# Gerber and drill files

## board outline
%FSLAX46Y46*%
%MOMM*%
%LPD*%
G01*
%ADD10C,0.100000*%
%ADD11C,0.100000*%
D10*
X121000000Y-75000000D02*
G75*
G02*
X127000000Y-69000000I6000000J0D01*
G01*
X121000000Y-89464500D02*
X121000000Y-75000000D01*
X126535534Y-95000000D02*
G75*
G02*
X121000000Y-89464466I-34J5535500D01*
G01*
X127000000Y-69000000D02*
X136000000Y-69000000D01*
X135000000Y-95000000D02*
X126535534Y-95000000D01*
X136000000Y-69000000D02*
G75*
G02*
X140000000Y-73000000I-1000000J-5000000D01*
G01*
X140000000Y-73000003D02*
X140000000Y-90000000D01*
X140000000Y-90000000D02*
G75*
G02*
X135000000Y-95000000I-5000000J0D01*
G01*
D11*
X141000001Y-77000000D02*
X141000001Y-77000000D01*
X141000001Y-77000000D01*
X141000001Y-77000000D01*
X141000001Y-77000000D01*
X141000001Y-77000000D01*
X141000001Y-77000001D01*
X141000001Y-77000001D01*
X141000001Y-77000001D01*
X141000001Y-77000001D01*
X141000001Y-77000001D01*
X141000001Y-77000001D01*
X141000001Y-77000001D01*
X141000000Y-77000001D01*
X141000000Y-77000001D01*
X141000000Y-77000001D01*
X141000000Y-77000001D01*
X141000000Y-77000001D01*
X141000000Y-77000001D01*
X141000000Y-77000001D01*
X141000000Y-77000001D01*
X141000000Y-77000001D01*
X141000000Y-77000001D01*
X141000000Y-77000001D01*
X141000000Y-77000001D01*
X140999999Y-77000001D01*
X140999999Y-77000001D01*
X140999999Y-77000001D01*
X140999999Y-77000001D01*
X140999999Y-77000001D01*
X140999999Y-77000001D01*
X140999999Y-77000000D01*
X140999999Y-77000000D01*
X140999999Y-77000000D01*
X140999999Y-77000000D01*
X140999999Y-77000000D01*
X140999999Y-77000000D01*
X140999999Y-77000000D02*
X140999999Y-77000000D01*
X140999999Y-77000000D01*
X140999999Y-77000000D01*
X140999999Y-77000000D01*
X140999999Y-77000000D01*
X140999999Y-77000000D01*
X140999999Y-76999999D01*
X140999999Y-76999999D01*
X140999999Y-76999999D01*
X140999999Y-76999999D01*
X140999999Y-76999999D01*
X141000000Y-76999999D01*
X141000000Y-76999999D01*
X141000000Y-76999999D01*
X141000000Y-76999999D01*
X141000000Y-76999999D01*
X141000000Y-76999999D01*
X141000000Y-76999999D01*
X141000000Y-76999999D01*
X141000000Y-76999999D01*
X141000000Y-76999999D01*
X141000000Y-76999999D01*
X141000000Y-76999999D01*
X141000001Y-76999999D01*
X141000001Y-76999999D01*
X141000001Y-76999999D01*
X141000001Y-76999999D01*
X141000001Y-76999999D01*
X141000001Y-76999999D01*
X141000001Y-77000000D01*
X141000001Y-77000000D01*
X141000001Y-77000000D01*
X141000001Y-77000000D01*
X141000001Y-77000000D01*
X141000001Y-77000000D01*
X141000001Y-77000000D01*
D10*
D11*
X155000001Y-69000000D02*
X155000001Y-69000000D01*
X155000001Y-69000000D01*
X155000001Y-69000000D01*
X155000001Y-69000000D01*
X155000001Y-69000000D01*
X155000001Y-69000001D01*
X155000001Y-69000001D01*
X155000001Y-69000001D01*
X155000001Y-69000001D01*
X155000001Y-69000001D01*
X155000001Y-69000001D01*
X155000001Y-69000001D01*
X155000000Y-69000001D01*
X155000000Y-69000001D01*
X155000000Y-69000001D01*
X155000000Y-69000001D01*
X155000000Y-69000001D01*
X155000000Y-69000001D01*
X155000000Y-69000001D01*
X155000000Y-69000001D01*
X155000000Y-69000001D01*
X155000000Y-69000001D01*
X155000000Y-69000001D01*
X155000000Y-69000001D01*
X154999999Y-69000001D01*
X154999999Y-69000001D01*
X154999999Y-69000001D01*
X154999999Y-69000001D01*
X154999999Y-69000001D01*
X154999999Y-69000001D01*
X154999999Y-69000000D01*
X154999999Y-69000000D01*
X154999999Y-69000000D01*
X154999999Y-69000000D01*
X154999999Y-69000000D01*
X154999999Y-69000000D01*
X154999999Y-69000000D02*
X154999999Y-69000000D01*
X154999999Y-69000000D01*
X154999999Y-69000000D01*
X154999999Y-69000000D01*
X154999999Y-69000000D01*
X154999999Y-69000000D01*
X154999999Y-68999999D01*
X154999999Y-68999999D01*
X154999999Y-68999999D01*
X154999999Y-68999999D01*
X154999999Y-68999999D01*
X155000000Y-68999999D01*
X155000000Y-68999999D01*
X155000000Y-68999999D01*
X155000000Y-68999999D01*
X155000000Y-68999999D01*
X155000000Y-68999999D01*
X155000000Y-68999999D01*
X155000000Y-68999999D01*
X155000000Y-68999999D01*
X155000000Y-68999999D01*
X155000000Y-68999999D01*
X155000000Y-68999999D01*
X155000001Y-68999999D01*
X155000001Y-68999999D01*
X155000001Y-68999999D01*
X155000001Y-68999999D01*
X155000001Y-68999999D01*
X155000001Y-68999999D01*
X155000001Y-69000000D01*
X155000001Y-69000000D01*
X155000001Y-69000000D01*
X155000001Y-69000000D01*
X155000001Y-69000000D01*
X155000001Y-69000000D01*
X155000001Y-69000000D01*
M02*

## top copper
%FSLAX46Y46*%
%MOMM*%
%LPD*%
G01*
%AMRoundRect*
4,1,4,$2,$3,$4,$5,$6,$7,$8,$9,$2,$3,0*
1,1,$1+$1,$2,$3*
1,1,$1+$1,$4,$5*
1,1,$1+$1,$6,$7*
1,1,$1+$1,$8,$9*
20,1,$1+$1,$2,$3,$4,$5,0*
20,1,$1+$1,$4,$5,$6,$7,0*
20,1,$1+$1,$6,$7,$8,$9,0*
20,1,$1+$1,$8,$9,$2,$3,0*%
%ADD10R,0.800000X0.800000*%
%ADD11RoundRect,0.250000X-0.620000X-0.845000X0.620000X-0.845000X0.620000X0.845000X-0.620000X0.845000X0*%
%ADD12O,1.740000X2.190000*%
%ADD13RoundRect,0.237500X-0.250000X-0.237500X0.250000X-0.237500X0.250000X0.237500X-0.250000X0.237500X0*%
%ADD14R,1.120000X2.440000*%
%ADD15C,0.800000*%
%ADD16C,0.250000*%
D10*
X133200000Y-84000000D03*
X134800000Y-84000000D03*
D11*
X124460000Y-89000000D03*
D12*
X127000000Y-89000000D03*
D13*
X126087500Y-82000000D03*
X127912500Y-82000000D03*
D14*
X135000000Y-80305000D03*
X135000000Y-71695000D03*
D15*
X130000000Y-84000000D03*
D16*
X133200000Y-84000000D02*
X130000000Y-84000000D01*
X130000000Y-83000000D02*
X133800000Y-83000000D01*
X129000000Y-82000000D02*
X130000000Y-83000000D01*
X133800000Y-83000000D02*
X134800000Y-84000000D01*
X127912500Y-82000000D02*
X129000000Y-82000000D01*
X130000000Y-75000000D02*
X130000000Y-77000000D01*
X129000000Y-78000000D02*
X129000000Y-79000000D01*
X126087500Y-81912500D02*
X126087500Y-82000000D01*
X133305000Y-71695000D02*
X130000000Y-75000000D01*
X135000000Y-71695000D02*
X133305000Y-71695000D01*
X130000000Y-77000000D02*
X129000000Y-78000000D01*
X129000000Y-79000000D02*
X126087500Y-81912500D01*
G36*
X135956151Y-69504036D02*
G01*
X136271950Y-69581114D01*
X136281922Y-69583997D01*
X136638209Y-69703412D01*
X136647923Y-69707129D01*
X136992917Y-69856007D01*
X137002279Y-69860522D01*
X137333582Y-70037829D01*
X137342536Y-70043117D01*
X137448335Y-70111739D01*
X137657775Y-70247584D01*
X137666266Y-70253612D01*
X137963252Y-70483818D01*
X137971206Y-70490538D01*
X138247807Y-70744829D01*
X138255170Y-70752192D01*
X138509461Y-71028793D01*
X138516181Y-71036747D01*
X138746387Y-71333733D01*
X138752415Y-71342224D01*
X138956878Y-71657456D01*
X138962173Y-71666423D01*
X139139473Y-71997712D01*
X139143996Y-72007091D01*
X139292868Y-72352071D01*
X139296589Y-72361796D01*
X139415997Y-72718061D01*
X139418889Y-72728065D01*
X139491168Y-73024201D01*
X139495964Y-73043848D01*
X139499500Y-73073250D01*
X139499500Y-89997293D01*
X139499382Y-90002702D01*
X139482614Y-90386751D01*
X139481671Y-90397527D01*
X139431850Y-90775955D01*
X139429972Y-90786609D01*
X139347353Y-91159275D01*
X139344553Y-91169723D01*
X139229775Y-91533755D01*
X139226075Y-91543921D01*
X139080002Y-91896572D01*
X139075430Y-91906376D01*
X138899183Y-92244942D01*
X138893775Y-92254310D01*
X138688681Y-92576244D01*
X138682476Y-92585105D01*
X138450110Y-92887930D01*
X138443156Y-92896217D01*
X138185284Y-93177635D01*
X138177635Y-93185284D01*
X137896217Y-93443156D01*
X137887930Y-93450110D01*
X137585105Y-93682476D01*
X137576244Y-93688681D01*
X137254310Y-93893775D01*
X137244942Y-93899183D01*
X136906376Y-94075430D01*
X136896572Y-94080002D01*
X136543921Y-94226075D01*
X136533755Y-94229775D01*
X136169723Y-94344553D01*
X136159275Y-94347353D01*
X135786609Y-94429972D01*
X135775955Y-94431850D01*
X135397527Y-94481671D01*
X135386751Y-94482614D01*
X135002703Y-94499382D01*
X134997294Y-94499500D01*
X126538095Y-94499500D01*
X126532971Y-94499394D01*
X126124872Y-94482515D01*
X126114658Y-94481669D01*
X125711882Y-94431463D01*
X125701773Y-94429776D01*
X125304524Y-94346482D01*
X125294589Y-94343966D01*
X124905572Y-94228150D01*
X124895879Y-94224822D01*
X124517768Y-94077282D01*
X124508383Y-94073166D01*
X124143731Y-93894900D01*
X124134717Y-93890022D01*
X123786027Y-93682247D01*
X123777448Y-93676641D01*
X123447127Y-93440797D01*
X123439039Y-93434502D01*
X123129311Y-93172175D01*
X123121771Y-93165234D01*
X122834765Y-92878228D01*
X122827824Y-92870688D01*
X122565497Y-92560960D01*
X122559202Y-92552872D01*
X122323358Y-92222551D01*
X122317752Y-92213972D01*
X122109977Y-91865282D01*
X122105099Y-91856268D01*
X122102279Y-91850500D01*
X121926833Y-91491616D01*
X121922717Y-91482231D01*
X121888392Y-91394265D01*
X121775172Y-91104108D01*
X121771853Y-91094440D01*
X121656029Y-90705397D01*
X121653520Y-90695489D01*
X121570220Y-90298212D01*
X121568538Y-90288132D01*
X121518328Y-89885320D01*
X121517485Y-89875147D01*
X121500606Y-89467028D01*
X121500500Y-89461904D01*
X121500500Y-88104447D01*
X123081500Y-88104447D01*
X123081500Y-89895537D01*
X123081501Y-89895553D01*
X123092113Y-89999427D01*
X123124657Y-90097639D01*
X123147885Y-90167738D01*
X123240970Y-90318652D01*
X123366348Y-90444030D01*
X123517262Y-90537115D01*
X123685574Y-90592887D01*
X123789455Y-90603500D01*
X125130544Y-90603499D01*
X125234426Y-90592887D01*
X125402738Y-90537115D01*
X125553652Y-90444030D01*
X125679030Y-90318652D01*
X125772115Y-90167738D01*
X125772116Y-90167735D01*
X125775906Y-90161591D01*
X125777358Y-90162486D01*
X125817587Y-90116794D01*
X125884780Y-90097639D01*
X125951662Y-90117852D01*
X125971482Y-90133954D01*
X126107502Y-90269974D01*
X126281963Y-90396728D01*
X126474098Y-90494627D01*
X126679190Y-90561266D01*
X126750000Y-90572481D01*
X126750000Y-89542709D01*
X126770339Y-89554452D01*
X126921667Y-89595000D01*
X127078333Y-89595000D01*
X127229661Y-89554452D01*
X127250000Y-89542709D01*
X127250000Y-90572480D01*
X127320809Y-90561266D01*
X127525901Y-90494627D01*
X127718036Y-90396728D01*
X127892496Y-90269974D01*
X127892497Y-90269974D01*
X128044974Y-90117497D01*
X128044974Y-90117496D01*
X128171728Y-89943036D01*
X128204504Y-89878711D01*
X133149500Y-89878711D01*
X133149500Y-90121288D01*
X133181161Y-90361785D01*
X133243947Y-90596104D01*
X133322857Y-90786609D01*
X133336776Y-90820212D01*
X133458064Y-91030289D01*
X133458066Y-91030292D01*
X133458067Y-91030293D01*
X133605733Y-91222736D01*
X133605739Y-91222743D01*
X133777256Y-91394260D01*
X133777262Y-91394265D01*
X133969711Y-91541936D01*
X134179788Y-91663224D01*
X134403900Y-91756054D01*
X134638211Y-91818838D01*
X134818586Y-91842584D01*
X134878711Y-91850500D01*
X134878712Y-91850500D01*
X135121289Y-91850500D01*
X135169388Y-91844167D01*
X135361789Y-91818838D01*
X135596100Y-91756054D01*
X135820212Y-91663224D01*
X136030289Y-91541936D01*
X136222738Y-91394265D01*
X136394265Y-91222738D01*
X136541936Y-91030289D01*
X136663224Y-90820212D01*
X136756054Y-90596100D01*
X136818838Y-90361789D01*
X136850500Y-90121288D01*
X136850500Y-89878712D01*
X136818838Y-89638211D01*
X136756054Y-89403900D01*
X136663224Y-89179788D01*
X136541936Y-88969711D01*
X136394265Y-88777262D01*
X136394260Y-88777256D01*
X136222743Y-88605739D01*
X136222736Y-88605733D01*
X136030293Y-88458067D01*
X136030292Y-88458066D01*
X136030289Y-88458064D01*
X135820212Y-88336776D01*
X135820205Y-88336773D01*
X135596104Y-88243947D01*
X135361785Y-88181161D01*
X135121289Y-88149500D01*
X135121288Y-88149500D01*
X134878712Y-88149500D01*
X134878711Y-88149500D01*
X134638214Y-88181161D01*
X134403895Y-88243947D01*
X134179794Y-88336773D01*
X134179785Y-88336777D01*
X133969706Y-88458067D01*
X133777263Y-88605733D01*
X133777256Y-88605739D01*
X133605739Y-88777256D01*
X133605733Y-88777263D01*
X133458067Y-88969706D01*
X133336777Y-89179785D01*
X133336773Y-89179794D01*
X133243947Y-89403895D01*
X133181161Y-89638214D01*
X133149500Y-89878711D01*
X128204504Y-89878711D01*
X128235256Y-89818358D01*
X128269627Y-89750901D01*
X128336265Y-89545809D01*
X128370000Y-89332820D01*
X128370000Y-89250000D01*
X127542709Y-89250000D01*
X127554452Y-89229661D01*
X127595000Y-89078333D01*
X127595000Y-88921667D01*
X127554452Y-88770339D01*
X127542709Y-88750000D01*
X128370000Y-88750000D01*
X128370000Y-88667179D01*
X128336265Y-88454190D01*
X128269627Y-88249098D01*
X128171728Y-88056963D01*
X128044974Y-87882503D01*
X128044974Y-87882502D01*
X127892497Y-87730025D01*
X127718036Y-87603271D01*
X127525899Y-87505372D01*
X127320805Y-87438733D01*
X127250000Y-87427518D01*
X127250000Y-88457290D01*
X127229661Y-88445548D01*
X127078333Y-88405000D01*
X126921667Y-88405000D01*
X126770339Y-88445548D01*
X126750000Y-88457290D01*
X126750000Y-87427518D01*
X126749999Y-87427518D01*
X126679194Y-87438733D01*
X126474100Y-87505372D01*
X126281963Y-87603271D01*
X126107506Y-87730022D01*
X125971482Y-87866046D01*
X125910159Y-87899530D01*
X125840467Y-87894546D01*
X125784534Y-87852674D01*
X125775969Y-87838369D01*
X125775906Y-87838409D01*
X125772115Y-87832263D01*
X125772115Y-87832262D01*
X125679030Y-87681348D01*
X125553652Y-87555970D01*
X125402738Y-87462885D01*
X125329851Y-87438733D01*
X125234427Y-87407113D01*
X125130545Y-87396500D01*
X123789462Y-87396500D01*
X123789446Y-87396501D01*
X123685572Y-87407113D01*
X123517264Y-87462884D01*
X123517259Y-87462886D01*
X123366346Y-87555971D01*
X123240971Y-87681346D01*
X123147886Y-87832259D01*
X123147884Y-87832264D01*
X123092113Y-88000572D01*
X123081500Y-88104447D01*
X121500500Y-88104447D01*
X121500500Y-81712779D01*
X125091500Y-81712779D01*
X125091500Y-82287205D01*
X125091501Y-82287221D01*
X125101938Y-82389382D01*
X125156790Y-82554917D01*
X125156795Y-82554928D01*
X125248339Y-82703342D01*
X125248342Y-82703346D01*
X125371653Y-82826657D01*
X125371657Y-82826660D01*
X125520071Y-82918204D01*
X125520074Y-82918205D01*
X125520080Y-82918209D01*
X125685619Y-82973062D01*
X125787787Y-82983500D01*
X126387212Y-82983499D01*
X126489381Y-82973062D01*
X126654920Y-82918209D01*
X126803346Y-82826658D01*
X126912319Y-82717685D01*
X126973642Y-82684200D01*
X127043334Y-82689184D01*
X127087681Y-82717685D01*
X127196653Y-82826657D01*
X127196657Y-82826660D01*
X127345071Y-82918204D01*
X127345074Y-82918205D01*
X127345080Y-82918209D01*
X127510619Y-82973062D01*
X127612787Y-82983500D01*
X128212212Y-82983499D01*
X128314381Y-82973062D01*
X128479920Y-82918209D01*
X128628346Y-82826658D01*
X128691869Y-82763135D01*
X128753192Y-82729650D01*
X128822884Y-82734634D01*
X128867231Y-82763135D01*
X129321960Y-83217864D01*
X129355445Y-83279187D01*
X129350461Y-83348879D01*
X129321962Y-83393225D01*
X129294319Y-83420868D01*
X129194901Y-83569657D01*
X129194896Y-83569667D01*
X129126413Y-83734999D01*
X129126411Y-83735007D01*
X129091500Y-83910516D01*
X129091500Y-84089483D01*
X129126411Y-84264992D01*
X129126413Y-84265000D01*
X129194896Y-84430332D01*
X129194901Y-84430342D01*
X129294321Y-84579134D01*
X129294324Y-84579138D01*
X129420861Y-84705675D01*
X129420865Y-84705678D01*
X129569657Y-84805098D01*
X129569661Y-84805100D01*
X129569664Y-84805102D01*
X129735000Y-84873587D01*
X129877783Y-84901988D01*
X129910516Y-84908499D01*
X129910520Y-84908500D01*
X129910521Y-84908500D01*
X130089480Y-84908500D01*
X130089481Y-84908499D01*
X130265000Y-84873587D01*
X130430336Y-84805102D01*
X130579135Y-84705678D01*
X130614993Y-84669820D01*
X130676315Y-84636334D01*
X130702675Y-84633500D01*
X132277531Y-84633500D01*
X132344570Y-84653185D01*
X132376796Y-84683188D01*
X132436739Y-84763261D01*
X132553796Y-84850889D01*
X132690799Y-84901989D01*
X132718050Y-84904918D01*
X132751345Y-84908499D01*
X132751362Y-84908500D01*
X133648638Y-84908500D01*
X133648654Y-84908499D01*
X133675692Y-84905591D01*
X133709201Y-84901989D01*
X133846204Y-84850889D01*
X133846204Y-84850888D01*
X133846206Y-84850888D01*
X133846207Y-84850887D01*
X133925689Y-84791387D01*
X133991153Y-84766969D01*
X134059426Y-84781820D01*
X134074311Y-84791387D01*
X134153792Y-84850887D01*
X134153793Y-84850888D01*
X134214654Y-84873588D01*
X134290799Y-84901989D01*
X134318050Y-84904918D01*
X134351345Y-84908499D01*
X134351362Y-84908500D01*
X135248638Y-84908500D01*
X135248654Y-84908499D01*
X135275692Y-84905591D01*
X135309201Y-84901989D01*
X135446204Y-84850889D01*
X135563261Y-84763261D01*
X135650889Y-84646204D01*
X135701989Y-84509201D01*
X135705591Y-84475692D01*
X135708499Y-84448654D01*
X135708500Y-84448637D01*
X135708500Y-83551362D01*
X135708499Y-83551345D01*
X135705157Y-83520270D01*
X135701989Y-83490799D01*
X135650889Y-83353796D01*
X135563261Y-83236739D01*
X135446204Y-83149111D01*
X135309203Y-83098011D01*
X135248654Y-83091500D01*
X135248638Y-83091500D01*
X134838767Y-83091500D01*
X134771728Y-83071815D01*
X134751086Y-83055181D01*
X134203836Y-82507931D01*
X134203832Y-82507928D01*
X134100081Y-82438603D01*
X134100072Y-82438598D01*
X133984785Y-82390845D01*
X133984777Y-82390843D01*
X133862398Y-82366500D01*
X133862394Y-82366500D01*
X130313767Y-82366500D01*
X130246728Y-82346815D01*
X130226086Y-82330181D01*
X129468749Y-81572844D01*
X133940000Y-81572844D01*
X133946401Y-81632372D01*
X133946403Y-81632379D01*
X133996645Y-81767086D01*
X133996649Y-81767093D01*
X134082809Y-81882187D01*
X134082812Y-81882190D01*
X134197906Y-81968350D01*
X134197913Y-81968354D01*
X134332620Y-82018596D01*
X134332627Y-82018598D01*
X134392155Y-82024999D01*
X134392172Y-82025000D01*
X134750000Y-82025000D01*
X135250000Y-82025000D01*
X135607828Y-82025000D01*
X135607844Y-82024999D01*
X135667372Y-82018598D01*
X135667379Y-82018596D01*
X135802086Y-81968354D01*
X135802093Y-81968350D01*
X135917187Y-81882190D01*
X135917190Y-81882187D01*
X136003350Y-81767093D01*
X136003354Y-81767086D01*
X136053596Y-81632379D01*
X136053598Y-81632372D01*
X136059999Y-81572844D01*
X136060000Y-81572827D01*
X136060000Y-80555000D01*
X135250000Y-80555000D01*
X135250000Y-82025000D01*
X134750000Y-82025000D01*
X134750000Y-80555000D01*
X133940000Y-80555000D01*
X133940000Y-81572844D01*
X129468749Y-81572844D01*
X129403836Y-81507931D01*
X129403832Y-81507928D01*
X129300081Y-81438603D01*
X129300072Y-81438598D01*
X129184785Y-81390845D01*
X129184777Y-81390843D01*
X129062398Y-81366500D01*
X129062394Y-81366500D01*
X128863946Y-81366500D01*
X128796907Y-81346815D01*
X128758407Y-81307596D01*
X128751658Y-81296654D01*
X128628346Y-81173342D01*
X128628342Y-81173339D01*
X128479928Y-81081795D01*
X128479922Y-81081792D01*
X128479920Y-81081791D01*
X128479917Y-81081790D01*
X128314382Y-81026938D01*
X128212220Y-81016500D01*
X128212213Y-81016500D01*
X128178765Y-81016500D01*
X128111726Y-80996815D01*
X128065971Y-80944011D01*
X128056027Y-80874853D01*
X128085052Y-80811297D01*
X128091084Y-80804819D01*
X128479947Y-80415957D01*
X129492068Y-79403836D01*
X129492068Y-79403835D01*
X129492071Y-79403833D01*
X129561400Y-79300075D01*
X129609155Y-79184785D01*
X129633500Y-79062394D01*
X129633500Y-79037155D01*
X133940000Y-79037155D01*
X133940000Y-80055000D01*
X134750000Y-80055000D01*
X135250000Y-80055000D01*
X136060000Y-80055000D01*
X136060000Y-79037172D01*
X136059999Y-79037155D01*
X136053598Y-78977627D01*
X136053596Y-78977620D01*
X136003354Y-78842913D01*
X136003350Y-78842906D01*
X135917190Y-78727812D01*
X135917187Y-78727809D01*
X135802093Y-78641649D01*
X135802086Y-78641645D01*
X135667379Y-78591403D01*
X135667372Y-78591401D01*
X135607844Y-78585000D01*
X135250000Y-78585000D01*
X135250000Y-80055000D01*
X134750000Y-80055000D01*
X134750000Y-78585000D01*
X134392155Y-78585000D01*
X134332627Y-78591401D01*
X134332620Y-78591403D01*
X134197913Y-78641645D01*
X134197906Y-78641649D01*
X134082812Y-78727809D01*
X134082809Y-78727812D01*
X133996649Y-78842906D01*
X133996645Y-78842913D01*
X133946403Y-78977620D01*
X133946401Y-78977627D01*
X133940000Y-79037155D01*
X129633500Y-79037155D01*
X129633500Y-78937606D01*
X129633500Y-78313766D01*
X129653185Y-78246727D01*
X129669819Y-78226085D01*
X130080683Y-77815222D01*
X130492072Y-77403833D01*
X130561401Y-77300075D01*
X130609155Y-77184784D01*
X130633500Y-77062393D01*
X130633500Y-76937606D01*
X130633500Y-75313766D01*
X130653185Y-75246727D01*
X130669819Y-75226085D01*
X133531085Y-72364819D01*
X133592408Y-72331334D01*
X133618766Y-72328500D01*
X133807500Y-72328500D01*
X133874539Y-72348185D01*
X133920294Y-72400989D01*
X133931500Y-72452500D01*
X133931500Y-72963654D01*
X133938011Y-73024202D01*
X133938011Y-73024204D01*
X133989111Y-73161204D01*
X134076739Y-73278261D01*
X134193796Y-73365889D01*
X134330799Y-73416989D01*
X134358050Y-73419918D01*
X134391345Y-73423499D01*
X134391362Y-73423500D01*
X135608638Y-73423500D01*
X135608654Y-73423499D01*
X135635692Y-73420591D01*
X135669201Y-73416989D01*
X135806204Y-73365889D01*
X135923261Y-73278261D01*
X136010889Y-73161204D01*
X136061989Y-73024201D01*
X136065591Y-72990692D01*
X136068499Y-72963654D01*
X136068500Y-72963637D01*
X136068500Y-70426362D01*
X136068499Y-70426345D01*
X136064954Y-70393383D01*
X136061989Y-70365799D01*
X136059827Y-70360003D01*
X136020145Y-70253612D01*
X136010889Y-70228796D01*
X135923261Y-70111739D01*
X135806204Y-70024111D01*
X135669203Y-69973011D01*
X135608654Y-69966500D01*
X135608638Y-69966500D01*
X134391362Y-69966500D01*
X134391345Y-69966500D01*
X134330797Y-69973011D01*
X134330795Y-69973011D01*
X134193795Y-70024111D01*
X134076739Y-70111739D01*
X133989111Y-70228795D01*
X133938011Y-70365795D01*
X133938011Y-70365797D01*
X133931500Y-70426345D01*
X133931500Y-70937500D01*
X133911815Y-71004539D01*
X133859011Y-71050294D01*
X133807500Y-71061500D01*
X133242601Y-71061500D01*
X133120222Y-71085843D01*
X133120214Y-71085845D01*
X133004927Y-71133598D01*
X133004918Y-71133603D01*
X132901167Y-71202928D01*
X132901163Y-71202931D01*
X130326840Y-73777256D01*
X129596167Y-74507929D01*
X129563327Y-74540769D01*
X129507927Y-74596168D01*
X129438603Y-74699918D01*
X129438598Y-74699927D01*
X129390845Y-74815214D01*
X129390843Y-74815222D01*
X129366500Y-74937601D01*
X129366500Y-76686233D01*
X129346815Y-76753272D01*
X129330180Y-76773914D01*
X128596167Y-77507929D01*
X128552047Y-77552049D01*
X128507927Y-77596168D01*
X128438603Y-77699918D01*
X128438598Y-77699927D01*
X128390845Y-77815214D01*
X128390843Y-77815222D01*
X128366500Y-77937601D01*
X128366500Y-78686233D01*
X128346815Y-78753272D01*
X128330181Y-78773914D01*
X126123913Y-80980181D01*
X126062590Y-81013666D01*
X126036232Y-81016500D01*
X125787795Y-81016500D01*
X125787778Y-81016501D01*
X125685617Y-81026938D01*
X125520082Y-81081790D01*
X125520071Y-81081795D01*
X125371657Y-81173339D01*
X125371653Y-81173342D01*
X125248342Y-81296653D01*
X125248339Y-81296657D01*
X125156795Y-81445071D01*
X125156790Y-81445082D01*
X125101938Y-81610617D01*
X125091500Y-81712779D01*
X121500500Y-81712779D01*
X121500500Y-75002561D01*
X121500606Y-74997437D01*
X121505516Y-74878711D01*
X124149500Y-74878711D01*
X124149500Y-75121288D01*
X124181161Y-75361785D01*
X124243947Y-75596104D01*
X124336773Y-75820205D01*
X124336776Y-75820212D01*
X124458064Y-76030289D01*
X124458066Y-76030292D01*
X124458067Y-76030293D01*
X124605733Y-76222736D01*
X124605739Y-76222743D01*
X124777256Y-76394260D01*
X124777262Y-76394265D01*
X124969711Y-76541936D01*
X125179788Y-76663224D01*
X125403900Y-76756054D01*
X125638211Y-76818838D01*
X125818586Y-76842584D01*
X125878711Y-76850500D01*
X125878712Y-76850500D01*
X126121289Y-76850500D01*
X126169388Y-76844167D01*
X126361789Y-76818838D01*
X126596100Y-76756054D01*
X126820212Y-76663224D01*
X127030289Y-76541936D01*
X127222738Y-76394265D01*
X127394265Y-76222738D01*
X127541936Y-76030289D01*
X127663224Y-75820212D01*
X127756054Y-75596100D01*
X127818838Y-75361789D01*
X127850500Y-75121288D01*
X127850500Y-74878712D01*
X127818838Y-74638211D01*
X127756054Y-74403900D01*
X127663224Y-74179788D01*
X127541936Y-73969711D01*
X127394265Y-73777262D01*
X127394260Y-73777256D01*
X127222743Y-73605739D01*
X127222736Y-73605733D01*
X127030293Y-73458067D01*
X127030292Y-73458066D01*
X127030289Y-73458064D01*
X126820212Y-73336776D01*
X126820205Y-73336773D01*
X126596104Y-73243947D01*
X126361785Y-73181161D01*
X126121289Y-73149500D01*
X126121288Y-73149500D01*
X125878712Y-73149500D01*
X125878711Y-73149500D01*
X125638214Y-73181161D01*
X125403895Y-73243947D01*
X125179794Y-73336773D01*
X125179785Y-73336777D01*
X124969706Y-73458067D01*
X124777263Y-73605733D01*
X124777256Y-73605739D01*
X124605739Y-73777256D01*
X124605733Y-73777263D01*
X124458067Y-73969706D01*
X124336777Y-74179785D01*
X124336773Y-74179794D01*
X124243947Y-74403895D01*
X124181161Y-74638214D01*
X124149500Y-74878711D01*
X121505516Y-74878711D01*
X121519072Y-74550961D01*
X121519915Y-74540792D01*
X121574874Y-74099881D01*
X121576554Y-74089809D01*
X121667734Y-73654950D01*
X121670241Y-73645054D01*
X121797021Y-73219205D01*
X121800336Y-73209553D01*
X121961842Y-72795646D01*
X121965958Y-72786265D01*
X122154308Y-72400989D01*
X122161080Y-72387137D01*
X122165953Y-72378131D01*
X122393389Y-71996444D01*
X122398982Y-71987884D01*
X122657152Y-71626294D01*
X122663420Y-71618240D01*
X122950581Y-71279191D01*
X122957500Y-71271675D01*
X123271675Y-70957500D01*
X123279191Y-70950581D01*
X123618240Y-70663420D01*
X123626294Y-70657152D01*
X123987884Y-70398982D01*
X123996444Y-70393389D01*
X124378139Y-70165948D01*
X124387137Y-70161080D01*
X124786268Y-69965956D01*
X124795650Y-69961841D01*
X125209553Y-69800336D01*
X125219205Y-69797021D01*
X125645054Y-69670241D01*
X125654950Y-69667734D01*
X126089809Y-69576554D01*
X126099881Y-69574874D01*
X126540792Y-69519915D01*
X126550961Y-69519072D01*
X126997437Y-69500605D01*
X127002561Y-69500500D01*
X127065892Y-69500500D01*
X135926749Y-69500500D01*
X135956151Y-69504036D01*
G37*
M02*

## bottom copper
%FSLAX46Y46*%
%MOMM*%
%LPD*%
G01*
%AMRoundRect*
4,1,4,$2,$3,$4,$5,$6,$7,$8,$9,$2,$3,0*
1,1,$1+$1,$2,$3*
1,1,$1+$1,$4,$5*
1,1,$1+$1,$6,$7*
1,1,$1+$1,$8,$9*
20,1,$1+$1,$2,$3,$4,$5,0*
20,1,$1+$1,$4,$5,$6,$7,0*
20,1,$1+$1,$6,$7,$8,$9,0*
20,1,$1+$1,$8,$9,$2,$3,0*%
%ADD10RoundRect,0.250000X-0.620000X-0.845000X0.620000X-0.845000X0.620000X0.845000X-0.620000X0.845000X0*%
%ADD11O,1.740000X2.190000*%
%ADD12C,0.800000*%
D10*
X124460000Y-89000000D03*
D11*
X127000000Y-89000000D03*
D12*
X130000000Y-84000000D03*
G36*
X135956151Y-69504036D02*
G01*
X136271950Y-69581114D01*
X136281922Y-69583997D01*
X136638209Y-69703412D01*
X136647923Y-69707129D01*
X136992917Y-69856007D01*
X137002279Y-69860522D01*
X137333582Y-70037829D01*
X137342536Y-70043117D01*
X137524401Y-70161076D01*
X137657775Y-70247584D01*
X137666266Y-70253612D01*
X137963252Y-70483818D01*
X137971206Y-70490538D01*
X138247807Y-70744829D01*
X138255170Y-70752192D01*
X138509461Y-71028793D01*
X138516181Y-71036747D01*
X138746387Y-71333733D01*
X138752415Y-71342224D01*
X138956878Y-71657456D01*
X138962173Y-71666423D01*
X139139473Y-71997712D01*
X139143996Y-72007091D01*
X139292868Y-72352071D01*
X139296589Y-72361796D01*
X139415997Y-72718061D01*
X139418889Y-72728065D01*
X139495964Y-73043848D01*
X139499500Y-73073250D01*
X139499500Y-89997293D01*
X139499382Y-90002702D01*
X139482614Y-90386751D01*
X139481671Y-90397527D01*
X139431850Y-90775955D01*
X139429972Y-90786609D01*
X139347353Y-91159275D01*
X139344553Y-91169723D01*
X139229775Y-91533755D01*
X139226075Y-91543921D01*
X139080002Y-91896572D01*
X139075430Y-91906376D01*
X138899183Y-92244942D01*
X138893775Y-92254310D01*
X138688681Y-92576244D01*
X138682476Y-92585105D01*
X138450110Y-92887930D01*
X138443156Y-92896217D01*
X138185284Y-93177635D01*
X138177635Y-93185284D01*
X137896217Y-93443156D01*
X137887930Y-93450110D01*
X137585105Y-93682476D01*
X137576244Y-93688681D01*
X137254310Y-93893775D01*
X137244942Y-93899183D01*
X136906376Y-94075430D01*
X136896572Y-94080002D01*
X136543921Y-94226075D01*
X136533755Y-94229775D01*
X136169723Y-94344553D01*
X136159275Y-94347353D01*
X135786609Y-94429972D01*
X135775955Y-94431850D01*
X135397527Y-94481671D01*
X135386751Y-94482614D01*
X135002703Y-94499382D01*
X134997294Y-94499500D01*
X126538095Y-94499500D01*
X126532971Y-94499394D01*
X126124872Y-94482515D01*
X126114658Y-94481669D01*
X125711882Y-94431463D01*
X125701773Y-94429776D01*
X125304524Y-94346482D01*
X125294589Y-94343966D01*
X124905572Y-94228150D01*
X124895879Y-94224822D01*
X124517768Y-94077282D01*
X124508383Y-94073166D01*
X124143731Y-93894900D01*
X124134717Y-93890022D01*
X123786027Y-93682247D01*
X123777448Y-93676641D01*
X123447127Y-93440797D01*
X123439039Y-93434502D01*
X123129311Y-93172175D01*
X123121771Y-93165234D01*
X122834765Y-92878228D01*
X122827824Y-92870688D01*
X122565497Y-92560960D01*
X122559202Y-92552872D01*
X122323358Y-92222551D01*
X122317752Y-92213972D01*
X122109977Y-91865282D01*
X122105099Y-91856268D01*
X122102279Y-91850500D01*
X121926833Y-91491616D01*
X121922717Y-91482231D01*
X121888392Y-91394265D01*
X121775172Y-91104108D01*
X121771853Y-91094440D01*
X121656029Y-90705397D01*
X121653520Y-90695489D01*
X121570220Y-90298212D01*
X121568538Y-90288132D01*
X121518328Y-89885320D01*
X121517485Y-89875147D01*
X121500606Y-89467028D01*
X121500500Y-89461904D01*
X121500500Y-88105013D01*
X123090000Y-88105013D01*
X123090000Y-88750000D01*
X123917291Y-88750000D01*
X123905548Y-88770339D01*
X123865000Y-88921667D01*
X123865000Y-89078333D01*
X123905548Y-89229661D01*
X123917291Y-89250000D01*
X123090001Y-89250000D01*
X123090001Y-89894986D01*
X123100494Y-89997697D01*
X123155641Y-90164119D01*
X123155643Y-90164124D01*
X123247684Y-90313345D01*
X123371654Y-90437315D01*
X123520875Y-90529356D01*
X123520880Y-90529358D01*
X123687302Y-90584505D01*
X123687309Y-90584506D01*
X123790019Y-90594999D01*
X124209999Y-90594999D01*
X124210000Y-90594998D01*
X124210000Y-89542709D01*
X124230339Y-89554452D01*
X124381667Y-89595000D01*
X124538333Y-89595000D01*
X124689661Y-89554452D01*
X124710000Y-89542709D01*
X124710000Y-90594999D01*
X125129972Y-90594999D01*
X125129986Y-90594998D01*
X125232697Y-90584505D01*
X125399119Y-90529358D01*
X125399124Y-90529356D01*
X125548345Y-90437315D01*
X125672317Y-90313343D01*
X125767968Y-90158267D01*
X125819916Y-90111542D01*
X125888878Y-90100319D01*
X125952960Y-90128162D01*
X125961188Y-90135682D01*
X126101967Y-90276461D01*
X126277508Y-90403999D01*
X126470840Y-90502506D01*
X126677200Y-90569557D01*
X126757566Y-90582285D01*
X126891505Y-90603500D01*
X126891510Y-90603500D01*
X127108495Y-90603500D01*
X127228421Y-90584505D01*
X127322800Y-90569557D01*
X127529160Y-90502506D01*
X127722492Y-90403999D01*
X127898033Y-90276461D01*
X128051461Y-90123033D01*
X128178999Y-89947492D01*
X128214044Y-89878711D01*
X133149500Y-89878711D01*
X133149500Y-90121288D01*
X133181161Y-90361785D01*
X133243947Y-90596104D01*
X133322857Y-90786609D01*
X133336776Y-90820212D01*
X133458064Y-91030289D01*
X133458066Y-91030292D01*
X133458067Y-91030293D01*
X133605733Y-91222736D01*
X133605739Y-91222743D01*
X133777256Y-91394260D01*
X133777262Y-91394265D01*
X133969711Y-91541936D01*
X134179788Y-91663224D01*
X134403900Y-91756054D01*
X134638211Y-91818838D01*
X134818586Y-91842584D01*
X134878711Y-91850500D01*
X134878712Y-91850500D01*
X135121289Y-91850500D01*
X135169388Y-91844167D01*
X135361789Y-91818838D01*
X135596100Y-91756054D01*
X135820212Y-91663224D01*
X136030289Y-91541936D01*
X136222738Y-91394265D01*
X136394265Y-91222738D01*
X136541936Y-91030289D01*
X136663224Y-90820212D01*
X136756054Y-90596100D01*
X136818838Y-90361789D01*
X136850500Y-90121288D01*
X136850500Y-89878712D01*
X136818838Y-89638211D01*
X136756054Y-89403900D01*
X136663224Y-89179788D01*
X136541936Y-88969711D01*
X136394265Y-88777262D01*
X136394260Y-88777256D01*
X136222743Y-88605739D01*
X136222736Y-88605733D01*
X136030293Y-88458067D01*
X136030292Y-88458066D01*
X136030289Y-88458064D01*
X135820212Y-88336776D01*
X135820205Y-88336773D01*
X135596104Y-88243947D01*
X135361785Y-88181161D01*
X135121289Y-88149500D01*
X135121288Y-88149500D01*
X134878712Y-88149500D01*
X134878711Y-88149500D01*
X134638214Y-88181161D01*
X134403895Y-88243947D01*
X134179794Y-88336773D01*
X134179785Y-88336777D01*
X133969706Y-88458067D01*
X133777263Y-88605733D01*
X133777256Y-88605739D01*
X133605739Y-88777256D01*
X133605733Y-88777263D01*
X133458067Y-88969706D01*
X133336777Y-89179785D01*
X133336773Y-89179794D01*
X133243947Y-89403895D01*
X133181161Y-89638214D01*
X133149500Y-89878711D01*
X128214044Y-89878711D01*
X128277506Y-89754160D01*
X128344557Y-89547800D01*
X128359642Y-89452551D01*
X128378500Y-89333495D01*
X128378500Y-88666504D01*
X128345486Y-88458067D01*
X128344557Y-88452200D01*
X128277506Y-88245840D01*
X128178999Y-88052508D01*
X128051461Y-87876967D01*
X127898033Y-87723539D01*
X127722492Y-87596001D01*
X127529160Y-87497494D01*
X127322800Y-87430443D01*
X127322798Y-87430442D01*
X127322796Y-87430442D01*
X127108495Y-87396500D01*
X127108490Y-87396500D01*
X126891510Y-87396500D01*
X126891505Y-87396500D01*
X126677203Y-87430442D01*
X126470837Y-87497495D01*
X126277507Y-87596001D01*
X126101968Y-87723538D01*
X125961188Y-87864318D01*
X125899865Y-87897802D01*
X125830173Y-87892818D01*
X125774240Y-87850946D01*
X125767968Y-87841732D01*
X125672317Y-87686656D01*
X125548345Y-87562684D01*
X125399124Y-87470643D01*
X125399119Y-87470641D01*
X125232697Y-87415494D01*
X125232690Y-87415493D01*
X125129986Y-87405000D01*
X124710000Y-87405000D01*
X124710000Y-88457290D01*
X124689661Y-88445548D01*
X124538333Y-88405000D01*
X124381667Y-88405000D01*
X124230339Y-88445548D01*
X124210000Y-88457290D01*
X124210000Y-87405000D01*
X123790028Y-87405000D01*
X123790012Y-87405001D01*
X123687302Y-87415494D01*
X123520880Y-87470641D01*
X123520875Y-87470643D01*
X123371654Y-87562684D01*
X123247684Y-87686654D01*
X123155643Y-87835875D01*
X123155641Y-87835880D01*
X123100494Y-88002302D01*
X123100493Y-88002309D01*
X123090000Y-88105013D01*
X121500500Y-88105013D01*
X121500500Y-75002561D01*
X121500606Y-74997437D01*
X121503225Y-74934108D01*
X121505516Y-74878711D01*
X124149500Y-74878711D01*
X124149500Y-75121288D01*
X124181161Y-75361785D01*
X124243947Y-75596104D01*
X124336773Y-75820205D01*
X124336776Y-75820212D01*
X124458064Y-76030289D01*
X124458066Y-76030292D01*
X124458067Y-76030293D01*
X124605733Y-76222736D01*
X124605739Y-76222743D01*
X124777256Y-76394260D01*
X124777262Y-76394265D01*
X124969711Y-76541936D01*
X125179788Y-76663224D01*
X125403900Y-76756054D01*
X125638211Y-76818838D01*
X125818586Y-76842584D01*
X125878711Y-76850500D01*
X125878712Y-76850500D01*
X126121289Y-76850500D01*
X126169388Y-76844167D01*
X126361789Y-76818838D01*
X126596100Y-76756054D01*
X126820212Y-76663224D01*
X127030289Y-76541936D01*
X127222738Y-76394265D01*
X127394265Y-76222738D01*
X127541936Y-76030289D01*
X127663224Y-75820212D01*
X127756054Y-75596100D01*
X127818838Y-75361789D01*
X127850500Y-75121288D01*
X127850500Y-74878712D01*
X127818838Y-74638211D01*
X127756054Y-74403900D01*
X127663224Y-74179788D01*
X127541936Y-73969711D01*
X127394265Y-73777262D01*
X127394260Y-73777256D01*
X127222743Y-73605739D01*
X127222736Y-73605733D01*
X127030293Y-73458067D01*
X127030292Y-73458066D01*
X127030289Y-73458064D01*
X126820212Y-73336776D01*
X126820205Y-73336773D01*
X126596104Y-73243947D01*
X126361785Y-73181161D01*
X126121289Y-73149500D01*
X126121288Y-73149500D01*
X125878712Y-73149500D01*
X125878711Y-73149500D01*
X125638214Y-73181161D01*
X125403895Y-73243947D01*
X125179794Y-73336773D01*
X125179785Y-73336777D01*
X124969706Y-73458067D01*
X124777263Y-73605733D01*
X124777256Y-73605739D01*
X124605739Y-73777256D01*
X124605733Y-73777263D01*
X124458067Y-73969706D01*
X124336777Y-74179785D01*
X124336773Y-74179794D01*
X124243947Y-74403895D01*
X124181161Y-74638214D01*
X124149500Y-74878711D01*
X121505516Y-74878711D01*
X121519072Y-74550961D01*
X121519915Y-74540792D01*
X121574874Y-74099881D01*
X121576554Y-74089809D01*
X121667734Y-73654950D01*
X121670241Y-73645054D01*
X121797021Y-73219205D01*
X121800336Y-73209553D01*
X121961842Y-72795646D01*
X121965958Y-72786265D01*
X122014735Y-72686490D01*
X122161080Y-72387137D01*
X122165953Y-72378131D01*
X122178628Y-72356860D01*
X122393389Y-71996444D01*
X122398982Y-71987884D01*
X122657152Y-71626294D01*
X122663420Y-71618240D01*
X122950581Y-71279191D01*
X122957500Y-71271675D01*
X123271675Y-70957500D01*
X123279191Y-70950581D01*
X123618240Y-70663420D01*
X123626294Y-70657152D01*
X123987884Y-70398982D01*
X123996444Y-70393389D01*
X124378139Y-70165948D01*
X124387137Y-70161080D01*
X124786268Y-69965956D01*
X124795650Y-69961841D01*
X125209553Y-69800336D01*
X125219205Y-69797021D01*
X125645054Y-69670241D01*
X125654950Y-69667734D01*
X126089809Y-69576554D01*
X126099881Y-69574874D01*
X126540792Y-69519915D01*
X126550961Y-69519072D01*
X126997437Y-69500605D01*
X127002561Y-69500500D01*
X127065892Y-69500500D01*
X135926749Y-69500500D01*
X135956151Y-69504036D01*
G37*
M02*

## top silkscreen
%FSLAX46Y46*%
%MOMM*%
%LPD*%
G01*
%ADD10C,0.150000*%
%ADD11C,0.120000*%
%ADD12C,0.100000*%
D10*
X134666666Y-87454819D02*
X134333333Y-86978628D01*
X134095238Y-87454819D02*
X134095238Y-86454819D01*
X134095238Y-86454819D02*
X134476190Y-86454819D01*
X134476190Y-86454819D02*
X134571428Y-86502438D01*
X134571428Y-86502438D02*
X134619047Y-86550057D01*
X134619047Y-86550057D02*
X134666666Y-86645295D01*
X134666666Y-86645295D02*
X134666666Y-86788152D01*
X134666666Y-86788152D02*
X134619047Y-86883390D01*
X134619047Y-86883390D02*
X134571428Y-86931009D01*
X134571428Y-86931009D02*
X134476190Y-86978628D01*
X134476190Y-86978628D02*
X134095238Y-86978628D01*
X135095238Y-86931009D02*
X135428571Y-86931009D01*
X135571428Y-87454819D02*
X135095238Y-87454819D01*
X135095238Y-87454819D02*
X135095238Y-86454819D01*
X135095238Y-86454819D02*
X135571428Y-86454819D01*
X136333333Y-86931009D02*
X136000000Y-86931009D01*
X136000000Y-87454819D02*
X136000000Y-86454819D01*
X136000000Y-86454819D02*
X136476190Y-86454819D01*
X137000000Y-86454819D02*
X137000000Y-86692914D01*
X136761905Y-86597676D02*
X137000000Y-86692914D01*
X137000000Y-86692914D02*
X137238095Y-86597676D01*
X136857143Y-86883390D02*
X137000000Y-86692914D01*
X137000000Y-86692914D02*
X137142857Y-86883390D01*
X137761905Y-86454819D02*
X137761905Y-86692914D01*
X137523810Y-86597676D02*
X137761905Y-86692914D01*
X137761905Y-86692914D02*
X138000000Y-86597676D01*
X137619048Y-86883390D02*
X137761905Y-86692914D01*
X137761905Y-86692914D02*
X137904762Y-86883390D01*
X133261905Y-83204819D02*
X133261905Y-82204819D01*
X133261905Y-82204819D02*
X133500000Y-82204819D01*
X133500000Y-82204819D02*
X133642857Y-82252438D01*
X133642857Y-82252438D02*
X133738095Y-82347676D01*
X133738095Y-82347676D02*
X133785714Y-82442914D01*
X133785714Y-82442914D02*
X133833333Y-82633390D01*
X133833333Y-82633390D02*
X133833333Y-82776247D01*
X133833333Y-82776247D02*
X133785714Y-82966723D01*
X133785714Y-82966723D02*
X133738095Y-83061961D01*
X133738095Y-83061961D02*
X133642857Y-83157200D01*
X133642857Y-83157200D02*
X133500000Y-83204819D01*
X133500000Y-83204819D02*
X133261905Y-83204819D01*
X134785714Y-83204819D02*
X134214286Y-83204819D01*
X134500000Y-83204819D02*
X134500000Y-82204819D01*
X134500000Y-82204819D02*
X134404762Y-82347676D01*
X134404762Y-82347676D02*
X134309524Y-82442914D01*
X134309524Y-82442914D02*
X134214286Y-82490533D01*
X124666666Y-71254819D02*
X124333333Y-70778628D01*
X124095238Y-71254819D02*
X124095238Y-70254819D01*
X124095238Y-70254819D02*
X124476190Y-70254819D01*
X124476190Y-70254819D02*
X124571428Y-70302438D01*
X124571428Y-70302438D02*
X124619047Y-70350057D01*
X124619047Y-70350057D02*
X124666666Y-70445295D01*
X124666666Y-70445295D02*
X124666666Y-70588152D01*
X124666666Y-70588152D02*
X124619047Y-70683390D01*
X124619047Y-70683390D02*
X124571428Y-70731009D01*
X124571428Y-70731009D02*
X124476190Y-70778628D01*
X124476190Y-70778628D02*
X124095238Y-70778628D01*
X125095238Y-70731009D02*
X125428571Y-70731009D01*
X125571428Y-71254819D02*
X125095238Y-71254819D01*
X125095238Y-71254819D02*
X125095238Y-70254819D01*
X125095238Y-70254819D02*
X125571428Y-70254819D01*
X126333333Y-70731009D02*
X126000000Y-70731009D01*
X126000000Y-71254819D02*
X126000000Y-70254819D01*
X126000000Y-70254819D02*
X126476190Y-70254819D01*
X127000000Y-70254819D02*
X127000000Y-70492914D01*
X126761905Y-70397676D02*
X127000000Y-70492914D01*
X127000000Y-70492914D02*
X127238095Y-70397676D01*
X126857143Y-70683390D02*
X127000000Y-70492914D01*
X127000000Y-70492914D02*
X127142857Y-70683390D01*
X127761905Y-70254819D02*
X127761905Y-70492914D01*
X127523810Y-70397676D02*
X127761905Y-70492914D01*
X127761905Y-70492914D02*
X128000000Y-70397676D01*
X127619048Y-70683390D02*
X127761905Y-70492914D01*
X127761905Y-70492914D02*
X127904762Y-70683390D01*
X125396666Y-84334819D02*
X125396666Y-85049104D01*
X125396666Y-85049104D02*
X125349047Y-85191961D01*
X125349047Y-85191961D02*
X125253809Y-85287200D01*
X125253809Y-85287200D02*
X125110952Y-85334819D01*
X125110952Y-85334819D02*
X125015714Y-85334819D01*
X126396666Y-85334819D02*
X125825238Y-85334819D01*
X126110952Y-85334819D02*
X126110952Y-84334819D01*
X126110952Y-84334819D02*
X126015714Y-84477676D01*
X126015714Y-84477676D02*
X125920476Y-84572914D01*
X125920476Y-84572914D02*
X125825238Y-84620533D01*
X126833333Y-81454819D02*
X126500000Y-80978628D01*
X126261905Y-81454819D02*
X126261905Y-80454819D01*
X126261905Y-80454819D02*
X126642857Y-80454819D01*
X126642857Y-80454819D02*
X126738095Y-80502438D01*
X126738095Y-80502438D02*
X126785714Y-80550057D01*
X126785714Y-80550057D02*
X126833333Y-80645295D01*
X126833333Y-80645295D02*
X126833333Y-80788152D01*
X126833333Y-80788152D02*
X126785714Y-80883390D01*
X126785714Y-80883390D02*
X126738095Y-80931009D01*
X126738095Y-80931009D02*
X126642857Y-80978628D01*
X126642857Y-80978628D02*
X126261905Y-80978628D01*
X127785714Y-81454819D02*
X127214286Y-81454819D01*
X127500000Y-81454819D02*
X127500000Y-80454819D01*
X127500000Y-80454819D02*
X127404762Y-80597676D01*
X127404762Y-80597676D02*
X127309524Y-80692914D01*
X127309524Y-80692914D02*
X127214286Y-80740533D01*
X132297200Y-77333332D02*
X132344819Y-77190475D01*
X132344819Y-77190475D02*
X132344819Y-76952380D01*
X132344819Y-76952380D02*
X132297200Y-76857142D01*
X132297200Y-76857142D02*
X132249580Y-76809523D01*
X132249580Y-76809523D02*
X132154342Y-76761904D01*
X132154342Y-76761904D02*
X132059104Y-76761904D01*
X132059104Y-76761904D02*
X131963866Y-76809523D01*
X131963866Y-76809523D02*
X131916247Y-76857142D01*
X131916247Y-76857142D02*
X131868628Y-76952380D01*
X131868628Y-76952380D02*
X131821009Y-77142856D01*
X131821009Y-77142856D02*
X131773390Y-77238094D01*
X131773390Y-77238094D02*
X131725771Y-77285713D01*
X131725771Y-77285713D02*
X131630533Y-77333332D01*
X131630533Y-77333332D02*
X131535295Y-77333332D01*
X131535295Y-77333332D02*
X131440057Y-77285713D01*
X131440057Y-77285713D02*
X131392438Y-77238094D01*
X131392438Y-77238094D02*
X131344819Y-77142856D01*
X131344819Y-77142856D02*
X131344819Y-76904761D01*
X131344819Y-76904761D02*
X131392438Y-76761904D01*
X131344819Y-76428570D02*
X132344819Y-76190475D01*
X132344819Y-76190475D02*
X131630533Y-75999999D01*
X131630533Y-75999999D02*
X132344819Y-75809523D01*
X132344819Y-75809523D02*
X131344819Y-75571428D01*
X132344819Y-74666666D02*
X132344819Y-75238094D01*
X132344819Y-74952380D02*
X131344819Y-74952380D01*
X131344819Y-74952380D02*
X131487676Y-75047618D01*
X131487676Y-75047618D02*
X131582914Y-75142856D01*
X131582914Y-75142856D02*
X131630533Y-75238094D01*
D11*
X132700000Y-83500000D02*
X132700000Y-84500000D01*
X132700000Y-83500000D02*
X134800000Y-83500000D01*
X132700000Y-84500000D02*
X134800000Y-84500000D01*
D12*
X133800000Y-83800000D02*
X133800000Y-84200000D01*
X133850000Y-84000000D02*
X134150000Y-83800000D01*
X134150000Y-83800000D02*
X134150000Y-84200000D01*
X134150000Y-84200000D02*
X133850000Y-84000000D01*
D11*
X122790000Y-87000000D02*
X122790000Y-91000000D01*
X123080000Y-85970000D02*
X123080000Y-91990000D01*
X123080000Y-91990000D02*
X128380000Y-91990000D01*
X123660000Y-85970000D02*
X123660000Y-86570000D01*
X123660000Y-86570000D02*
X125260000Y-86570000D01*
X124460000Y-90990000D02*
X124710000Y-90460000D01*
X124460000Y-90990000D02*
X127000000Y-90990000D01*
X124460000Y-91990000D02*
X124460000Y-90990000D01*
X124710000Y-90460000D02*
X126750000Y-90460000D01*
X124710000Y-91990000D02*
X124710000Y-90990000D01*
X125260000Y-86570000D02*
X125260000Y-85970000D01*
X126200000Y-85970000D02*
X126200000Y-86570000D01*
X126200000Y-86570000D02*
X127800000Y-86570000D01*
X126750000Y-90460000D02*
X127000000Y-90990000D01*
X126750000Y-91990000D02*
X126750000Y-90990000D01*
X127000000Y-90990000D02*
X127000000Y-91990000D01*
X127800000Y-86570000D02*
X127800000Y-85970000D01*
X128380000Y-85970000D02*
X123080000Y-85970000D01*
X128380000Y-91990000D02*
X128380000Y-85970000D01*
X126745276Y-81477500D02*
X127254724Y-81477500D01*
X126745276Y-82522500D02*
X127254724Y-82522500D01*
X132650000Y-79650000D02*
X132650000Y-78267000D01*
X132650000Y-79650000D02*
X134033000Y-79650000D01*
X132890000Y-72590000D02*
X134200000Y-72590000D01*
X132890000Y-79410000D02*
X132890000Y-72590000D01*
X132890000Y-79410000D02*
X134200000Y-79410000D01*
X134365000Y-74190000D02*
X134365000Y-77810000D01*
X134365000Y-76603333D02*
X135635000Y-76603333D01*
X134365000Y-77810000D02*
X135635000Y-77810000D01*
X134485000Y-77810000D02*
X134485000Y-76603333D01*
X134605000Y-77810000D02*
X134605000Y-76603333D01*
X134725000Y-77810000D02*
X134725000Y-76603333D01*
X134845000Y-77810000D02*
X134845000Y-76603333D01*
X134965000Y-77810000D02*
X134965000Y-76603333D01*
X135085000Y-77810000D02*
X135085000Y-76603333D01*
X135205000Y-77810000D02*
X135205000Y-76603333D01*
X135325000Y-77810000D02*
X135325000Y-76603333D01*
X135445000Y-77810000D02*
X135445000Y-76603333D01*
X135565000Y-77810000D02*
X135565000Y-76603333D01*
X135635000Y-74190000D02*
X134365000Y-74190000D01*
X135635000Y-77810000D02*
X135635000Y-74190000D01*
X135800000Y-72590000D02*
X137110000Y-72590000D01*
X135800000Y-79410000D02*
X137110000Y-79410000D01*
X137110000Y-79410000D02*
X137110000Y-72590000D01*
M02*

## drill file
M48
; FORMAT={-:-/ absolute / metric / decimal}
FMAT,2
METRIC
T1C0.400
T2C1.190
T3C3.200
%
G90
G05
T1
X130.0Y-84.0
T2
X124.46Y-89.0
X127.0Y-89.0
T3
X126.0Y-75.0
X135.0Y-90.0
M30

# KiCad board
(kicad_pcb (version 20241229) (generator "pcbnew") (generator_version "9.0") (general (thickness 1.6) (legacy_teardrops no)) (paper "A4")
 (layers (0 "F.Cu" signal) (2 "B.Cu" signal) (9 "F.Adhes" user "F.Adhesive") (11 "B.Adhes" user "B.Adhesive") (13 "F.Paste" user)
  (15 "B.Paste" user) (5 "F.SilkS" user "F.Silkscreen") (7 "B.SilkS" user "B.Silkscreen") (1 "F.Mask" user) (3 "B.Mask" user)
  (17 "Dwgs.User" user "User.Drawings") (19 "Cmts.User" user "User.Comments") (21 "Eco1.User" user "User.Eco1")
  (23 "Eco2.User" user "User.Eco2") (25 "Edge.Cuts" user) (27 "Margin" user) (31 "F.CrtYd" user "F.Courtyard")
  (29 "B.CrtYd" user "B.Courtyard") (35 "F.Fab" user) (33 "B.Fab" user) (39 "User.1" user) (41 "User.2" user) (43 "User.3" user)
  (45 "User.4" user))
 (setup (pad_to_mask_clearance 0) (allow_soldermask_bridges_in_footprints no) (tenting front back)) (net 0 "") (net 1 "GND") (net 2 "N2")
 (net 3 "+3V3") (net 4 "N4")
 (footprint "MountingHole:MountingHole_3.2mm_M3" (layer "F.Cu") (at 135 90)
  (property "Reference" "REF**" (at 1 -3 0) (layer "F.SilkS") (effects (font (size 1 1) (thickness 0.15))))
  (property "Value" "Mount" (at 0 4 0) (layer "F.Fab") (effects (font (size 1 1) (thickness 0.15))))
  (pad "" np_thru_hole circle (at 0 0) (size 3.2 3.2) (drill 3.2) (layers "*.Cu" "*.Mask")))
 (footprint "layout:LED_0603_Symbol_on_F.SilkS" (layer "F.Cu") (at 134 84)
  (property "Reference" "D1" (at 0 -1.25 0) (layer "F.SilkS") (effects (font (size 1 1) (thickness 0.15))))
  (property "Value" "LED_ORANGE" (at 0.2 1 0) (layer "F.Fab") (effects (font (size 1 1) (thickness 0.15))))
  (fp_line (start -1.3 -0.5) (end -1.3 0.5) (stroke (width 0.12) (type solid)) (layer "F.SilkS"))
  (fp_line (start -1.3 -0.5) (end 0.8 -0.5) (stroke (width 0.12) (type solid)) (layer "F.SilkS"))
  (fp_line (start -1.3 0.5) (end 0.8 0.5) (stroke (width 0.12) (type solid)) (layer "F.SilkS"))
  (fp_line (start -0.2 -0.2) (end -0.2 0.2) (stroke (width 0.1) (type solid)) (layer "F.SilkS"))
  (fp_line (start -0.15 0) (end 0.15 -0.2) (stroke (width 0.1) (type solid)) (layer "F.SilkS"))
  (fp_line (start 0.15 -0.2) (end 0.15 0.2) (stroke (width 0.1) (type solid)) (layer "F.SilkS"))
  (fp_line (start 0.15 0.2) (end -0.15 0) (stroke (width 0.1) (type solid)) (layer "F.SilkS"))
  (pad "1" smd rect (at -0.8 0 180) (size 0.8 0.8) (layers "F.Cu" "F.Mask" "F.Paste") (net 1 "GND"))
  (pad "2" smd rect (at 0.8 0 180) (size 0.8 0.8) (layers "F.Cu" "F.Mask" "F.Paste") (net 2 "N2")))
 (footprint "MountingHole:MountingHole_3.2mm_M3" (layer "F.Cu") (at 126 75)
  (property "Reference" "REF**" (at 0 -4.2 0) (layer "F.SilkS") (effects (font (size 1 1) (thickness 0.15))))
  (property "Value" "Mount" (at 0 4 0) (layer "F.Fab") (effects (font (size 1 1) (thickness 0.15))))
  (pad "" np_thru_hole circle (at 0 0) (size 3.2 3.2) (drill 3.2) (layers "*.Cu" "*.Mask")))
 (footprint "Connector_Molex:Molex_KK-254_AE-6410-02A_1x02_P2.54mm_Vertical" (layer "F.Cu") (at 124.46 89)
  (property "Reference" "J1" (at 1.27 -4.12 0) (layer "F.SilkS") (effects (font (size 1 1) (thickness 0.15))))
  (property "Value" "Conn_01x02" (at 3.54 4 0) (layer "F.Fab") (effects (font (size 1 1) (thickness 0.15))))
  (fp_line (start -1.67 -2) (end -1.67 2) (stroke (width 0.12) (type solid)) (layer "F.SilkS"))
  (fp_line (start -1.38 -3.03) (end -1.38 2.99) (stroke (width 0.12) (type solid)) (layer "F.SilkS"))
  (fp_line (start -1.38 2.99) (end 3.92 2.99) (stroke (width 0.12) (type solid)) (layer "F.SilkS"))
  (fp_line (start -0.8 -3.03) (end -0.8 -2.43) (stroke (width 0.12) (type solid)) (layer "F.SilkS"))
  (fp_line (start -0.8 -2.43) (end 0.8 -2.43) (stroke (width 0.12) (type solid)) (layer "F.SilkS"))
  (fp_line (start 0 1.99) (end 0.25 1.46) (stroke (width 0.12) (type solid)) (layer "F.SilkS"))
  (fp_line (start 0 1.99) (end 2.54 1.99) (stroke (width 0.12) (type solid)) (layer "F.SilkS"))
  (fp_line (start 0 2.99) (end 0 1.99) (stroke (width 0.12) (type solid)) (layer "F.SilkS"))
  (fp_line (start 0.25 1.46) (end 2.29 1.46) (stroke (width 0.12) (type solid)) (layer "F.SilkS"))
  (fp_line (start 0.25 2.99) (end 0.25 1.99) (stroke (width 0.12) (type solid)) (layer "F.SilkS"))
  (fp_line (start 0.8 -2.43) (end 0.8 -3.03) (stroke (width 0.12) (type solid)) (layer "F.SilkS"))
  (fp_line (start 1.74 -3.03) (end 1.74 -2.43) (stroke (width 0.12) (type solid)) (layer "F.SilkS"))
  (fp_line (start 1.74 -2.43) (end 3.34 -2.43) (stroke (width 0.12) (type solid)) (layer "F.SilkS"))
  (fp_line (start 2.29 1.46) (end 2.54 1.99) (stroke (width 0.12) (type solid)) (layer "F.SilkS"))
  (fp_line (start 2.29 2.99) (end 2.29 1.99) (stroke (width 0.12) (type solid)) (layer "F.SilkS"))
  (fp_line (start 2.54 1.99) (end 2.54 2.99) (stroke (width 0.12) (type solid)) (layer "F.SilkS"))
  (fp_line (start 3.34 -2.43) (end 3.34 -3.03) (stroke (width 0.12) (type solid)) (layer "F.SilkS"))
  (fp_line (start 3.92 -3.03) (end -1.38 -3.03) (stroke (width 0.12) (type solid)) (layer "F.SilkS"))
  (fp_line (start 3.92 2.99) (end 3.92 -3.03) (stroke (width 0.12) (type solid)) (layer "F.SilkS"))
  (pad "1" thru_hole roundrect (at 0 0) (size 1.74 2.19) (drill 1.19) (layers "*.Cu" "*.Mask") (remove_unused_layers no)
   (roundrect_rratio 0.143678) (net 1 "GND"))
  (pad "2" thru_hole oval (at 2.54 0) (size 1.74 2.19) (drill 1.19) (layers "*.Cu" "*.Mask") (remove_unused_layers no) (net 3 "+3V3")))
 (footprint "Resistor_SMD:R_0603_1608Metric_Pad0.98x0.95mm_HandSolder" (layer "F.Cu") (at 127 82)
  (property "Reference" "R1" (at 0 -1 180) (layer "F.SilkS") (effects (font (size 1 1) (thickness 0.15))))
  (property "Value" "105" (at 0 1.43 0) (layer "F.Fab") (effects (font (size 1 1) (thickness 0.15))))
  (fp_line (start -0.254724 -0.5225) (end 0.254724 -0.5225) (stroke (width 0.12) (type solid)) (layer "F.SilkS"))
  (fp_line (start -0.254724 0.5225) (end 0.254724 0.5225) (stroke (width 0.12) (type solid)) (layer "F.SilkS"))
  (pad "1" smd roundrect (at -0.9125 0) (size 0.975 0.95) (layers "F.Cu" "F.Mask" "F.Paste") (roundrect_rratio 0.25) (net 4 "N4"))
  (pad "2" smd roundrect (at 0.9125 0) (size 0.975 0.95) (layers "F.Cu" "F.Mask" "F.Paste") (roundrect_rratio 0.25) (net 2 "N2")))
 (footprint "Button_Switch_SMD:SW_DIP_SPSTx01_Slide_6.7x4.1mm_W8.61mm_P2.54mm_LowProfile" (layer "F.Cu") (at 135 76 90)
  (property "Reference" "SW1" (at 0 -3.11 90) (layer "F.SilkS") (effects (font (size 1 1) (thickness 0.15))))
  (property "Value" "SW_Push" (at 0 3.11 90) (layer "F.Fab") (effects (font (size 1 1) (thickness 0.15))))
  (fp_line (start -3.65 -2.35) (end -2.267 -2.35) (stroke (width 0.12) (type solid)) (layer "F.SilkS"))
  (fp_line (start -3.65 -2.35) (end -3.65 -0.967) (stroke (width 0.12) (type solid)) (layer "F.SilkS"))
  (fp_line (start 3.41 -2.11) (end 3.41 -0.8) (stroke (width 0.12) (type solid)) (layer "F.SilkS"))
  (fp_line (start -3.41 -2.11) (end 3.41 -2.11) (stroke (width 0.12) (type solid)) (layer "F.SilkS"))
  (fp_line (start -3.41 -2.11) (end -3.41 -0.8) (stroke (width 0.12) (type solid)) (layer "F.SilkS"))
  (fp_line (start 1.81 -0.635) (end -1.81 -0.635) (stroke (width 0.12) (type solid)) (layer "F.SilkS"))
  (fp_line (start -0.603333 -0.635) (end -0.603333 0.635) (stroke (width 0.12) (type solid)) (layer "F.SilkS"))
  (fp_line (start -1.81 -0.635) (end -1.81 0.635) (stroke (width 0.12) (type solid)) (layer "F.SilkS"))
  (fp_line (start -1.81 -0.515) (end -0.603333 -0.515) (stroke (width 0.12) (type solid)) (layer "F.SilkS"))
  (fp_line (start -1.81 -0.395) (end -0.603333 -0.395) (stroke (width 0.12) (type solid)) (layer "F.SilkS"))
  (fp_line (start -1.81 -0.275) (end -0.603333 -0.275) (stroke (width 0.12) (type solid)) (layer "F.SilkS"))
  (fp_line (start -1.81 -0.155) (end -0.603333 -0.155) (stroke (width 0.12) (type solid)) (layer "F.SilkS"))
  (fp_line (start -1.81 -0.035) (end -0.603333 -0.035) (stroke (width 0.12) (type solid)) (layer "F.SilkS"))
  (fp_line (start -1.81 0.085) (end -0.603333 0.085) (stroke (width 0.12) (type solid)) (layer "F.SilkS"))
  (fp_line (start -1.81 0.205) (end -0.603333 0.205) (stroke (width 0.12) (type solid)) (layer "F.SilkS"))
  (fp_line (start -1.81 0.325) (end -0.603333 0.325) (stroke (width 0.12) (type solid)) (layer "F.SilkS"))
  (fp_line (start -1.81 0.445) (end -0.603333 0.445) (stroke (width 0.12) (type solid)) (layer "F.SilkS"))
  (fp_line (start -1.81 0.565) (end -0.603333 0.565) (stroke (width 0.12) (type solid)) (layer "F.SilkS"))
  (fp_line (start 1.81 0.635) (end 1.81 -0.635) (stroke (width 0.12) (type solid)) (layer "F.SilkS"))
  (fp_line (start -1.81 0.635) (end 1.81 0.635) (stroke (width 0.12) (type solid)) (layer "F.SilkS"))
  (fp_line (start 3.41 0.8) (end 3.41 2.11) (stroke (width 0.12) (type solid)) (layer "F.SilkS"))
  (fp_line (start -3.41 0.8) (end -3.41 2.11) (stroke (width 0.12) (type solid)) (layer "F.SilkS"))
  (fp_line (start -3.41 2.11) (end 3.41 2.11) (stroke (width 0.12) (type solid)) (layer "F.SilkS"))
  (pad "1" smd rect (at -4.305 0 90) (size 2.44 1.12) (layers "F.Cu" "F.Mask" "F.Paste") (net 3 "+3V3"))
  (pad "2" smd rect (at 4.305 0 90) (size 2.44 1.12) (layers "F.Cu" "F.Mask" "F.Paste") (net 4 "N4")))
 (gr_arc (start 121 75) (mid 122.757359 70.757359) (end 127 69) (stroke (width 0.1) (type default)) (layer "Edge.Cuts"))
 (gr_line (start 121 89.4645) (end 121 75) (stroke (width 0.1) (type default)) (layer "Edge.Cuts"))
 (gr_arc (start 126.535534 95) (mid 122.62132 93.37868) (end 121 89.464466) (stroke (width 0.1) (type default)) (layer "Edge.Cuts"))
 (gr_line (start 127 69) (end 136 69) (stroke (width 0.1) (type default)) (layer "Edge.Cuts"))
 (gr_line (start 135 95) (end 126.535534 95) (stroke (width 0.1) (type default)) (layer "Edge.Cuts"))
 (gr_arc (start 136 69) (mid 138.605551 70.394449) (end 140 73) (stroke (width 0.1) (type default)) (layer "Edge.Cuts"))
 (gr_line (start 140 73.000003) (end 140 90) (stroke (width 0.1) (type default)) (layer "Edge.Cuts"))
 (gr_arc (start 140 90) (mid 138.535534 93.535534) (end 135 95) (stroke (width 0.1) (type default)) (layer "Edge.Cuts"))
 (gr_arc (start 141 77) (mid 141 77) (end 141 77) (stroke (width 0.1) (type default)) (layer "Edge.Cuts"))
 (gr_arc (start 155 69) (mid 155 69) (end 155 69) (stroke (width 0.1) (type default)) (layer "Edge.Cuts"))
 (segment (start 133.2 84) (end 130 84) (width 0.25) (layer "F.Cu") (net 1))
 (via (at 130 84) (size 0.8) (drill 0.4) (layers "F.Cu" "B.Cu") (free yes) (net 1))
 (segment (start 130 83) (end 133.8 83) (width 0.25) (layer "F.Cu") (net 2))
 (segment (start 129 82) (end 130 83) (width 0.25) (layer "F.Cu") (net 2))
 (segment (start 133.8 83) (end 134.8 84) (width 0.25) (layer "F.Cu") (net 2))
 (segment (start 127.9125 82) (end 129 82) (width 0.25) (layer "F.Cu") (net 2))
 (segment (start 130 75) (end 130 77) (width 0.25) (layer "F.Cu") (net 4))
 (segment (start 129 78) (end 129 79) (width 0.25) (layer "F.Cu") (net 4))
 (segment (start 126.0875 81.9125) (end 126.0875 82) (width 0.25) (layer "F.Cu") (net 4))
 (segment (start 133.305 71.695) (end 130 75) (width 0.25) (layer "F.Cu") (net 4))
 (segment (start 135 71.695) (end 133.305 71.695) (width 0.25) (layer "F.Cu") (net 4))
 (segment (start 130 77) (end 129 78) (width 0.25) (layer "F.Cu") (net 4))
 (segment (start 129 79) (end 126.0875 81.9125) (width 0.25) (layer "F.Cu") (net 4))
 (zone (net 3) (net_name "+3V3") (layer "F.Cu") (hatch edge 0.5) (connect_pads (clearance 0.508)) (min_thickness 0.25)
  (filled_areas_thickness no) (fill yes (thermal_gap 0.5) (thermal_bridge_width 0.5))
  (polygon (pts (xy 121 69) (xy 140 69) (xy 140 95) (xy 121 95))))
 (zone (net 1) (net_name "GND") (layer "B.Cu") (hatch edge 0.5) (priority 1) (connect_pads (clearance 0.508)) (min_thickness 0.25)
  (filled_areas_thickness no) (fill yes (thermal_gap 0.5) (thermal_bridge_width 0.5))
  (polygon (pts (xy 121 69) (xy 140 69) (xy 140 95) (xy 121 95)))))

